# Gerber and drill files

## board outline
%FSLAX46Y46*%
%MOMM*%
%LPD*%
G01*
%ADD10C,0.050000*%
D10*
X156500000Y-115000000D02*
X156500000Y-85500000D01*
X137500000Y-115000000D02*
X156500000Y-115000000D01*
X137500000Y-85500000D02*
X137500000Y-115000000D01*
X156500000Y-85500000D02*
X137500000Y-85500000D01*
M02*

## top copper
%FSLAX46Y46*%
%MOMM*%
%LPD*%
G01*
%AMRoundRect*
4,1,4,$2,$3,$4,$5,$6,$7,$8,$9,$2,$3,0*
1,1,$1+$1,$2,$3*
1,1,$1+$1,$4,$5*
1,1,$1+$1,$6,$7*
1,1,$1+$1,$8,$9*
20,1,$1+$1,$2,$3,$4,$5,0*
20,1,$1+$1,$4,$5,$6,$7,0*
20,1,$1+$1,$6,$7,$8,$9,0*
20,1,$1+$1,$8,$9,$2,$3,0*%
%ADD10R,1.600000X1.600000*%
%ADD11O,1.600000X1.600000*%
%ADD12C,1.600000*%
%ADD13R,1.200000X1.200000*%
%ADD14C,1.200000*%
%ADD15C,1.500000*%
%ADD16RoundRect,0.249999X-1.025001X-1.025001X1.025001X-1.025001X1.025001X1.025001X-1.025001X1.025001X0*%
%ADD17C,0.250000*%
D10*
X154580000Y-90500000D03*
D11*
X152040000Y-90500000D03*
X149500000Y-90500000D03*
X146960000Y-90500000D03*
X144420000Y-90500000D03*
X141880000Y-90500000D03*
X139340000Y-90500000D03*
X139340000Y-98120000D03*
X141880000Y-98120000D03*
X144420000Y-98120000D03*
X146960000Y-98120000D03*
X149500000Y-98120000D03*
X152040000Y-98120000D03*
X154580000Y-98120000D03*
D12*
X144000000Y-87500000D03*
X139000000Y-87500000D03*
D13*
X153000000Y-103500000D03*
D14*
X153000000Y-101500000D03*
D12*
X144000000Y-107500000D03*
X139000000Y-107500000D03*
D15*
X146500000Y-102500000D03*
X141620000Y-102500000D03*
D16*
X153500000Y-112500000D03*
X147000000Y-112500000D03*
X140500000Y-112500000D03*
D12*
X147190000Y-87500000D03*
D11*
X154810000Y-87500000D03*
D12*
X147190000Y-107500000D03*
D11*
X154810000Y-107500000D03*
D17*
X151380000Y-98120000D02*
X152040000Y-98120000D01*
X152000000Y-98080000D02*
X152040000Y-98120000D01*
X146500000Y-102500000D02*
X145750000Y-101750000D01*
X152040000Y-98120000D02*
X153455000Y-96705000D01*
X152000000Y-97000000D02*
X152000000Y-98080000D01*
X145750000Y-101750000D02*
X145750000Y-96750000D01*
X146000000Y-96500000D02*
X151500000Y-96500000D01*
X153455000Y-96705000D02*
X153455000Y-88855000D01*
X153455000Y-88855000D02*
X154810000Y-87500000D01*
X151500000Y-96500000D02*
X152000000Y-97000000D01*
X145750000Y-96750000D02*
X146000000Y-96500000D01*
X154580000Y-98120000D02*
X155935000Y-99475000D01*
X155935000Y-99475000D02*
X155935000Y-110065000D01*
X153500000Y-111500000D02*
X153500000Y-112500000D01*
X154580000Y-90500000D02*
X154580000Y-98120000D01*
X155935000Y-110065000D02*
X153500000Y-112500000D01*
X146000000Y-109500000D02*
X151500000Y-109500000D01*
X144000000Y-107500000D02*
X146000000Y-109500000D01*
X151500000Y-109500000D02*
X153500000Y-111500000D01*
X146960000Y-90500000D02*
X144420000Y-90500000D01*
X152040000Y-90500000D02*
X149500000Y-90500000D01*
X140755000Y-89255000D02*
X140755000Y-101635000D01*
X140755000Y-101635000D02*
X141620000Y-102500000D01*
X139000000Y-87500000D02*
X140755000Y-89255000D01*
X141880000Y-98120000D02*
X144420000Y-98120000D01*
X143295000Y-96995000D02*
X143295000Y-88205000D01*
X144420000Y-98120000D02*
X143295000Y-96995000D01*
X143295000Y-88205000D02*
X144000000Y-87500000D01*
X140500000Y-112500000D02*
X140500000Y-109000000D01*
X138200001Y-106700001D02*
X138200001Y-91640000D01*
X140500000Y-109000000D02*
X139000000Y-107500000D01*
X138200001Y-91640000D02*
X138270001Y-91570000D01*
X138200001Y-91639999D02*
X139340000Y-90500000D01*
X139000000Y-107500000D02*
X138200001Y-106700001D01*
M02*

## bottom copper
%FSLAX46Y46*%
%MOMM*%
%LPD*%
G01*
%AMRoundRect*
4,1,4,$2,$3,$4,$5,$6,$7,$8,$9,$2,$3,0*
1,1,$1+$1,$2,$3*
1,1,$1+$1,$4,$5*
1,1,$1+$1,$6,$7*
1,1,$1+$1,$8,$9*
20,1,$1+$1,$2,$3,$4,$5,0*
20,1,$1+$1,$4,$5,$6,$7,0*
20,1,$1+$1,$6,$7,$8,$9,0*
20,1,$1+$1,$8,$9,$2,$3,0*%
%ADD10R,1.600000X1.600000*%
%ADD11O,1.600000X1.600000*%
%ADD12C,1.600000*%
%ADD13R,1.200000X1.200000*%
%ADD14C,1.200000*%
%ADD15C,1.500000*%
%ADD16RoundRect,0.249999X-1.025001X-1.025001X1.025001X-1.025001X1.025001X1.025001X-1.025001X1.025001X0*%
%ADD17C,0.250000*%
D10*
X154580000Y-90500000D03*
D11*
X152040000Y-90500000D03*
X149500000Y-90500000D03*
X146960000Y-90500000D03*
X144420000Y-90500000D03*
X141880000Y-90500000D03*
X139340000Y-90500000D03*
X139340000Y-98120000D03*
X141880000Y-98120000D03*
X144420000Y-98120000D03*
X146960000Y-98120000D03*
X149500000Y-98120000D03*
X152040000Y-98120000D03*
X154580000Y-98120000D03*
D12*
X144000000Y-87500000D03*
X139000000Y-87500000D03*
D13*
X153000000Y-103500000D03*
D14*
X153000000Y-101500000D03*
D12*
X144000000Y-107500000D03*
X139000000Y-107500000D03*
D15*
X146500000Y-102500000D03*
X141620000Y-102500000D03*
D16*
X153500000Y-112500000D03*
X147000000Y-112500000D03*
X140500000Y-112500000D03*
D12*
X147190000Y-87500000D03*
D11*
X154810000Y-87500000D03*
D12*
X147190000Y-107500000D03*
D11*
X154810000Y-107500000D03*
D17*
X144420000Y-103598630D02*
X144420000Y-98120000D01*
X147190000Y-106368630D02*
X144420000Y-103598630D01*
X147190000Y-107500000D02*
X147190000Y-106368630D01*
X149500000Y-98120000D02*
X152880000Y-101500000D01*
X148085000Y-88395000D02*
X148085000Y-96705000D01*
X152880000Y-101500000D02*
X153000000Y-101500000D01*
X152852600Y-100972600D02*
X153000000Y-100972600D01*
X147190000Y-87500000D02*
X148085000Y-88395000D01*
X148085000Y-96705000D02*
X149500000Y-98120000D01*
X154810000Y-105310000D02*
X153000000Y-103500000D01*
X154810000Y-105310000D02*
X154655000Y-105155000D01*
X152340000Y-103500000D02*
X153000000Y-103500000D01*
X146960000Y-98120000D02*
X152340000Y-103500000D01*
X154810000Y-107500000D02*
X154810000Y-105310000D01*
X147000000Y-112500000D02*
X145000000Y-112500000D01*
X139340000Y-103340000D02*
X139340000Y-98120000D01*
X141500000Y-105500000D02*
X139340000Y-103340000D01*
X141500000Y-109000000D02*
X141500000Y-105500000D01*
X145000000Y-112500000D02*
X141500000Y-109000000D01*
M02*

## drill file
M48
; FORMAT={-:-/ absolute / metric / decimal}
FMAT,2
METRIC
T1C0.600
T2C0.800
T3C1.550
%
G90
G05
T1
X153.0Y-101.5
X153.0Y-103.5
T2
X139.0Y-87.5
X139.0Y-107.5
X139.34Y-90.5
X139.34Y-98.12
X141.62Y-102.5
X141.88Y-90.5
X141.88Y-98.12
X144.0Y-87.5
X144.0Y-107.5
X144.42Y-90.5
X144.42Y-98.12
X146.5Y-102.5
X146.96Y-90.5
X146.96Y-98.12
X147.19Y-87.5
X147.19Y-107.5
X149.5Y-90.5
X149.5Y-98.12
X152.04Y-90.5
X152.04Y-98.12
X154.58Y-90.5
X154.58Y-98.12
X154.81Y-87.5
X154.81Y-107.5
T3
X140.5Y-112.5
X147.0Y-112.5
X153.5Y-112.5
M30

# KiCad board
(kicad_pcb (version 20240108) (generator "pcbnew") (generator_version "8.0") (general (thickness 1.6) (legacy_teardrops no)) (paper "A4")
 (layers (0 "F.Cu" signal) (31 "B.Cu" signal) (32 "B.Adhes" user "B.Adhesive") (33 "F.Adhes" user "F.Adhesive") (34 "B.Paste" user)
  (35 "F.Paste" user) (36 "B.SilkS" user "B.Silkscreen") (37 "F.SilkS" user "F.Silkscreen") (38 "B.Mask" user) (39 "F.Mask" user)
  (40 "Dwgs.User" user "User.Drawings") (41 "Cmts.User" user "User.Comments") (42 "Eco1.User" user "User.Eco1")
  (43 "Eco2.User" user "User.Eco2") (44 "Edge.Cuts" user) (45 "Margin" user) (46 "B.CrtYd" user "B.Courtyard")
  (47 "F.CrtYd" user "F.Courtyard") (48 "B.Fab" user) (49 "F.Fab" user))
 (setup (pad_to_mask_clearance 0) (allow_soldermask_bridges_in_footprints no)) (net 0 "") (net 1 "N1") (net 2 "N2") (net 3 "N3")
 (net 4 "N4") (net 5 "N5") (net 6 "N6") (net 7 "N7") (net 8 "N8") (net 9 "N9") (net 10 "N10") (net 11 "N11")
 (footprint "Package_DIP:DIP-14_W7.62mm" (layer "F.Cu") (at 154.58 90.5 -90)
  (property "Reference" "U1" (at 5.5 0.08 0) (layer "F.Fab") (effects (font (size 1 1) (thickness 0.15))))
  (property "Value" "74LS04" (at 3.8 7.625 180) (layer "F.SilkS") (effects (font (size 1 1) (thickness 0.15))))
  (pad "1" thru_hole rect (at 0 0 270) (size 1.6 1.6) (drill 0.8) (layers "*.Cu" "*.Mask") (remove_unused_layers no) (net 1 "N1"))
  (pad "2" thru_hole oval (at 0 2.54 270) (size 1.6 1.6) (drill 0.8) (layers "*.Cu" "*.Mask") (remove_unused_layers no) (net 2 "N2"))
  (pad "3" thru_hole oval (at 0 5.08 270) (size 1.6 1.6) (drill 0.8) (layers "*.Cu" "*.Mask") (remove_unused_layers no) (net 2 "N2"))
  (pad "4" thru_hole oval (at 0 7.62 270) (size 1.6 1.6) (drill 0.8) (layers "*.Cu" "*.Mask") (remove_unused_layers no) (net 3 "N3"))
  (pad "5" thru_hole oval (at 0 10.16 270) (size 1.6 1.6) (drill 0.8) (layers "*.Cu" "*.Mask") (remove_unused_layers no) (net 3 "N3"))
  (pad "6" thru_hole oval (at 0 12.7 270) (size 1.6 1.6) (drill 0.8) (layers "*.Cu" "*.Mask") (remove_unused_layers no) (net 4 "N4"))
  (pad "7" thru_hole oval (at 0 15.24 270) (size 1.6 1.6) (drill 0.8) (layers "*.Cu" "*.Mask") (remove_unused_layers no) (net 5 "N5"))
  (pad "8" thru_hole oval (at 7.62 15.24 270) (size 1.6 1.6) (drill 0.8) (layers "*.Cu" "*.Mask") (remove_unused_layers no) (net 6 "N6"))
  (pad "9" thru_hole oval (at 7.62 12.7 270) (size 1.6 1.6) (drill 0.8) (layers "*.Cu" "*.Mask") (remove_unused_layers no) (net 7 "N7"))
  (pad "10" thru_hole oval (at 7.62 10.16 270) (size 1.6 1.6) (drill 0.8) (layers "*.Cu" "*.Mask") (remove_unused_layers no) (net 7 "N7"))
  (pad "11" thru_hole oval (at 7.62 7.62 270) (size 1.6 1.6) (drill 0.8) (layers "*.Cu" "*.Mask") (remove_unused_layers no) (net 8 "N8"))
  (pad "12" thru_hole oval (at 7.62 5.08 270) (size 1.6 1.6) (drill 0.8) (layers "*.Cu" "*.Mask") (remove_unused_layers no) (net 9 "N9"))
  (pad "13" thru_hole oval (at 7.62 2.54 270) (size 1.6 1.6) (drill 0.8) (layers "*.Cu" "*.Mask") (remove_unused_layers no) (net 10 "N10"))
  (pad "14" thru_hole oval (at 7.62 0 270) (size 1.6 1.6) (drill 0.8) (layers "*.Cu" "*.Mask") (remove_unused_layers no) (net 1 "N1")))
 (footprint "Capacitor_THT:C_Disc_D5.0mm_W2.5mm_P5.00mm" (layer "F.Cu") (at 144 87.5 180)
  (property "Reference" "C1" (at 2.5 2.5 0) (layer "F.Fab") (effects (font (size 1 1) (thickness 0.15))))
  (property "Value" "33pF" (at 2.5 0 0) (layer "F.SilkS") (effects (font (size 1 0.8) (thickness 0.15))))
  (pad "1" thru_hole circle (at 0 0 180) (size 1.6 1.6) (drill 0.8) (layers "*.Cu" "*.Mask") (remove_unused_layers no) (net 7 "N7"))
  (pad "2" thru_hole circle (at 5 0 180) (size 1.6 1.6) (drill 0.8) (layers "*.Cu" "*.Mask") (remove_unused_layers no) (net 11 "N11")))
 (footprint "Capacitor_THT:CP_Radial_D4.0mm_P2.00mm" (layer "F.Cu") (at 153 103.5 90)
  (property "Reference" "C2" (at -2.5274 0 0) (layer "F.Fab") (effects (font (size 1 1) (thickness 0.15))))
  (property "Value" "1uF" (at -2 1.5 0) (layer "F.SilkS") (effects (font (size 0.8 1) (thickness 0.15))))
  (pad "1" thru_hole rect (at 0 0 90) (size 1.2 1.2) (drill 0.6) (layers "*.Cu" "*.Mask") (remove_unused_layers no) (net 8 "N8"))
  (pad "2" thru_hole circle (at 2 0 90) (size 1.2 1.2) (drill 0.6) (layers "*.Cu" "*.Mask") (remove_unused_layers no) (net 9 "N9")))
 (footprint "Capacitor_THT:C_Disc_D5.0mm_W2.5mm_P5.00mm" (layer "F.Cu") (at 144 107.5 180)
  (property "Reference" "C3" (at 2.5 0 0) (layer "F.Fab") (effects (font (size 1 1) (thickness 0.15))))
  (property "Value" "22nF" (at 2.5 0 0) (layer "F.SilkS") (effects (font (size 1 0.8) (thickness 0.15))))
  (pad "1" thru_hole circle (at 0 0 180) (size 1.6 1.6) (drill 0.8) (layers "*.Cu" "*.Mask") (remove_unused_layers no) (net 1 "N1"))
  (pad "2" thru_hole circle (at 5 0 180) (size 1.6 1.6) (drill 0.8) (layers "*.Cu" "*.Mask") (remove_unused_layers no) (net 5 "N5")))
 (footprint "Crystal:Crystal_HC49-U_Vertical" (layer "F.Cu") (at 146.5 102.5 180)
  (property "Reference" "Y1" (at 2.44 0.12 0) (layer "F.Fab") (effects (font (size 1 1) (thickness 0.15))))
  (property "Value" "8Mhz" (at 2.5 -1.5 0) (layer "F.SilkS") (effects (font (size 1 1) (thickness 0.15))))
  (pad "1" thru_hole circle (at 0 0 180) (size 1.5 1.5) (drill 0.8) (layers "*.Cu" "*.Mask") (remove_unused_layers no) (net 10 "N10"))
  (pad "2" thru_hole circle (at 4.88 0 180) (size 1.5 1.5) (drill 0.8) (layers "*.Cu" "*.Mask") (remove_unused_layers no) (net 11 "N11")))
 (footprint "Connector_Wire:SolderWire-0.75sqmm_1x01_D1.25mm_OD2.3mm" (layer "F.Cu") (at 153.5 112.5)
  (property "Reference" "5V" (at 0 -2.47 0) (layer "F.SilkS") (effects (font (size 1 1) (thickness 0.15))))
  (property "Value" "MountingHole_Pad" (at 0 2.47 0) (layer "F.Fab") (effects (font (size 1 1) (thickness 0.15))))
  (pad "1" thru_hole roundrect (at 0 0) (size 2.55 2.55) (drill 1.55) (layers "*.Cu" "*.Mask") (remove_unused_layers no)
   (roundrect_rratio 0.098039) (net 1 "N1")))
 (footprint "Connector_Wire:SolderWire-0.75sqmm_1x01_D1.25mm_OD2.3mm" (layer "F.Cu") (at 147 112.5)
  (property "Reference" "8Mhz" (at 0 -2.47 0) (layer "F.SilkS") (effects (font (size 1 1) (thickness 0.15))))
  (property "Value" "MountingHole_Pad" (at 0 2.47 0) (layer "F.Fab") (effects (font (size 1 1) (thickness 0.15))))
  (pad "1" thru_hole roundrect (at 0 0) (size 2.55 2.55) (drill 1.55) (layers "*.Cu" "*.Mask") (remove_unused_layers no)
   (roundrect_rratio 0.098039) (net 6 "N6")))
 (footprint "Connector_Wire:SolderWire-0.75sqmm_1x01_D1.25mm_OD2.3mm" (layer "F.Cu") (at 140.5 112.5)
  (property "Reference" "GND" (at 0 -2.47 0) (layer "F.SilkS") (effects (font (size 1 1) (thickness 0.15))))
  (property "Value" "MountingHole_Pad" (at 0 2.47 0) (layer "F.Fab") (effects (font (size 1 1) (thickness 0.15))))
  (pad "1" thru_hole roundrect (at 0 0) (size 2.55 2.55) (drill 1.55) (layers "*.Cu" "*.Mask") (remove_unused_layers no)
   (roundrect_rratio 0.098039) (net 5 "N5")))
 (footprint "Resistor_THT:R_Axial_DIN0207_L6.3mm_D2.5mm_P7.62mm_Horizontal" (layer "F.Cu") (at 147.19 87.5)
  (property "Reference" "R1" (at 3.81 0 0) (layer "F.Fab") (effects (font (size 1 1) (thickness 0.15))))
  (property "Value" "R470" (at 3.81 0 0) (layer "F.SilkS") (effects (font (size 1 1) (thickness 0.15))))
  (pad "1" thru_hole circle (at 0 0) (size 1.6 1.6) (drill 0.8) (layers "*.Cu" "*.Mask") (remove_unused_layers no) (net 9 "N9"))
  (pad "2" thru_hole oval (at 7.62 0) (size 1.6 1.6) (drill 0.8) (layers "*.Cu" "*.Mask") (remove_unused_layers no) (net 10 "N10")))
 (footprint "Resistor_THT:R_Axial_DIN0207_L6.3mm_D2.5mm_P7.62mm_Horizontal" (layer "F.Cu") (at 147.19 107.5)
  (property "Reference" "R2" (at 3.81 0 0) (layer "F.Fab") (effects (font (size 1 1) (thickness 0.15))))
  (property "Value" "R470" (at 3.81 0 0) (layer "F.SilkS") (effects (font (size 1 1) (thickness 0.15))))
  (pad "1" thru_hole circle (at 0 0) (size 1.6 1.6) (drill 0.8) (layers "*.Cu" "*.Mask") (remove_unused_layers no) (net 7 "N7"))
  (pad "2" thru_hole oval (at 7.62 0) (size 1.6 1.6) (drill 0.8) (layers "*.Cu" "*.Mask") (remove_unused_layers no) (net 8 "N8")))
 (gr_line (start 156.5 115) (end 156.5 85.5) (stroke (width 0.05) (type solid)) (layer "Edge.Cuts"))
 (gr_line (start 137.5 115) (end 156.5 115) (stroke (width 0.05) (type solid)) (layer "Edge.Cuts"))
 (gr_line (start 137.5 85.5) (end 137.5 115) (stroke (width 0.05) (type solid)) (layer "Edge.Cuts"))
 (gr_line (start 156.5 85.5) (end 137.5 85.5) (stroke (width 0.05) (type solid)) (layer "Edge.Cuts"))
 (segment (start 151.38 98.12) (end 152.04 98.12) (width 0.25) (layer "F.Cu") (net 10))
 (segment (start 152 98.08) (end 152.04 98.12) (width 0.25) (layer "F.Cu") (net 10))
 (segment (start 146.5 102.5) (end 145.75 101.75) (width 0.25) (layer "F.Cu") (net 10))
 (segment (start 152.04 98.12) (end 153.455 96.705) (width 0.25) (layer "F.Cu") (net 10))
 (segment (start 152 97) (end 152 98.08) (width 0.25) (layer "F.Cu") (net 10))
 (segment (start 145.75 101.75) (end 145.75 96.75) (width 0.25) (layer "F.Cu") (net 10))
 (segment (start 146 96.5) (end 151.5 96.5) (width 0.25) (layer "F.Cu") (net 10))
 (segment (start 153.455 96.705) (end 153.455 88.855) (width 0.25) (layer "F.Cu") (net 10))
 (segment (start 153.455 88.855) (end 154.81 87.5) (width 0.25) (layer "F.Cu") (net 10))
 (segment (start 151.5 96.5) (end 152 97) (width 0.25) (layer "F.Cu") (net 10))
 (segment (start 145.75 96.75) (end 146 96.5) (width 0.25) (layer "F.Cu") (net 10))
 (segment (start 154.58 98.12) (end 155.935 99.475) (width 0.25) (layer "F.Cu") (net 1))
 (segment (start 155.935 99.475) (end 155.935 110.065) (width 0.25) (layer "F.Cu") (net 1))
 (segment (start 153.5 111.5) (end 153.5 112.5) (width 0.25) (layer "F.Cu") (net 1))
 (segment (start 154.58 90.5) (end 154.58 98.12) (width 0.25) (layer "F.Cu") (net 1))
 (segment (start 155.935 110.065) (end 153.5 112.5) (width 0.25) (layer "F.Cu") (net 1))
 (segment (start 146 109.5) (end 151.5 109.5) (width 0.25) (layer "F.Cu") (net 1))
 (segment (start 144 107.5) (end 146 109.5) (width 0.25) (layer "F.Cu") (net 1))
 (segment (start 151.5 109.5) (end 153.5 111.5) (width 0.25) (layer "F.Cu") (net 1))
 (segment (start 146.96 90.5) (end 144.42 90.5) (width 0.25) (layer "F.Cu") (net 3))
 (segment (start 152.04 90.5) (end 149.5 90.5) (width 0.25) (layer "F.Cu") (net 2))
 (segment (start 140.755 89.255) (end 140.755 101.635) (width 0.25) (layer "F.Cu") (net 11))
 (segment (start 140.755 101.635) (end 141.62 102.5) (width 0.25) (layer "F.Cu") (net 11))
 (segment (start 139 87.5) (end 140.755 89.255) (width 0.25) (layer "F.Cu") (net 11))
 (segment (start 141.88 98.12) (end 144.42 98.12) (width 0.25) (layer "F.Cu") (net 7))
 (segment (start 143.295 96.995) (end 143.295 88.205) (width 0.25) (layer "F.Cu") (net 7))
 (segment (start 144.42 98.12) (end 143.295 96.995) (width 0.25) (layer "F.Cu") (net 7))
 (segment (start 143.295 88.205) (end 144 87.5) (width 0.25) (layer "F.Cu") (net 7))
 (segment (start 144.42 103.59863) (end 144.42 98.12) (width 0.25) (layer "B.Cu") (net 7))
 (segment (start 147.19 106.36863) (end 144.42 103.59863) (width 0.25) (layer "B.Cu") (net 7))
 (segment (start 147.19 107.5) (end 147.19 106.36863) (width 0.25) (layer "B.Cu") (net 7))
 (segment (start 149.5 98.12) (end 152.88 101.5) (width 0.25) (layer "B.Cu") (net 9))
 (segment (start 148.085 88.395) (end 148.085 96.705) (width 0.25) (layer "B.Cu") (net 9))
 (segment (start 152.88 101.5) (end 153 101.5) (width 0.25) (layer "B.Cu") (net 9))
 (segment (start 152.8526 100.9726) (end 153 100.9726) (width 0.25) (layer "B.Cu") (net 9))
 (segment (start 147.19 87.5) (end 148.085 88.395) (width 0.25) (layer "B.Cu") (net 9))
 (segment (start 148.085 96.705) (end 149.5 98.12) (width 0.25) (layer "B.Cu") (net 9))
 (segment (start 154.81 105.31) (end 153 103.5) (width 0.25) (layer "B.Cu") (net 8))
 (segment (start 154.81 105.31) (end 154.655 105.155) (width 0.25) (layer "B.Cu") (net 8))
 (segment (start 152.34 103.5) (end 153 103.5) (width 0.25) (layer "B.Cu") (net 8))
 (segment (start 146.96 98.12) (end 152.34 103.5) (width 0.25) (layer "B.Cu") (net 8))
 (segment (start 154.81 107.5) (end 154.81 105.31) (width 0.25) (layer "B.Cu") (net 8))
 (segment (start 147 112.5) (end 145 112.5) (width 0.25) (layer "B.Cu") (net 6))
 (segment (start 139.34 103.34) (end 139.34 98.12) (width 0.25) (layer "B.Cu") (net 6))
 (segment (start 141.5 105.5) (end 139.34 103.34) (width 0.25) (layer "B.Cu") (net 6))
 (segment (start 141.5 109) (end 141.5 105.5) (width 0.25) (layer "B.Cu") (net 6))
 (segment (start 145 112.5) (end 141.5 109) (width 0.25) (layer "B.Cu") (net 6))
 (segment (start 140.5 112.5) (end 140.5 109) (width 0.25) (layer "F.Cu") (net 5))
 (segment (start 138.200001 106.700001) (end 138.200001 91.64) (width 0.25) (layer "F.Cu") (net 5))
 (segment (start 140.5 109) (end 139 107.5) (width 0.25) (layer "F.Cu") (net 5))
 (segment (start 138.200001 91.64) (end 138.270001 91.57) (width 0.25) (layer "F.Cu") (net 5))
 (segment (start 138.200001 91.639999) (end 139.34 90.5) (width 0.25) (layer "F.Cu") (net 5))
 (segment (start 139 107.5) (end 138.200001 106.700001) (width 0.25) (layer "F.Cu") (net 5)))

